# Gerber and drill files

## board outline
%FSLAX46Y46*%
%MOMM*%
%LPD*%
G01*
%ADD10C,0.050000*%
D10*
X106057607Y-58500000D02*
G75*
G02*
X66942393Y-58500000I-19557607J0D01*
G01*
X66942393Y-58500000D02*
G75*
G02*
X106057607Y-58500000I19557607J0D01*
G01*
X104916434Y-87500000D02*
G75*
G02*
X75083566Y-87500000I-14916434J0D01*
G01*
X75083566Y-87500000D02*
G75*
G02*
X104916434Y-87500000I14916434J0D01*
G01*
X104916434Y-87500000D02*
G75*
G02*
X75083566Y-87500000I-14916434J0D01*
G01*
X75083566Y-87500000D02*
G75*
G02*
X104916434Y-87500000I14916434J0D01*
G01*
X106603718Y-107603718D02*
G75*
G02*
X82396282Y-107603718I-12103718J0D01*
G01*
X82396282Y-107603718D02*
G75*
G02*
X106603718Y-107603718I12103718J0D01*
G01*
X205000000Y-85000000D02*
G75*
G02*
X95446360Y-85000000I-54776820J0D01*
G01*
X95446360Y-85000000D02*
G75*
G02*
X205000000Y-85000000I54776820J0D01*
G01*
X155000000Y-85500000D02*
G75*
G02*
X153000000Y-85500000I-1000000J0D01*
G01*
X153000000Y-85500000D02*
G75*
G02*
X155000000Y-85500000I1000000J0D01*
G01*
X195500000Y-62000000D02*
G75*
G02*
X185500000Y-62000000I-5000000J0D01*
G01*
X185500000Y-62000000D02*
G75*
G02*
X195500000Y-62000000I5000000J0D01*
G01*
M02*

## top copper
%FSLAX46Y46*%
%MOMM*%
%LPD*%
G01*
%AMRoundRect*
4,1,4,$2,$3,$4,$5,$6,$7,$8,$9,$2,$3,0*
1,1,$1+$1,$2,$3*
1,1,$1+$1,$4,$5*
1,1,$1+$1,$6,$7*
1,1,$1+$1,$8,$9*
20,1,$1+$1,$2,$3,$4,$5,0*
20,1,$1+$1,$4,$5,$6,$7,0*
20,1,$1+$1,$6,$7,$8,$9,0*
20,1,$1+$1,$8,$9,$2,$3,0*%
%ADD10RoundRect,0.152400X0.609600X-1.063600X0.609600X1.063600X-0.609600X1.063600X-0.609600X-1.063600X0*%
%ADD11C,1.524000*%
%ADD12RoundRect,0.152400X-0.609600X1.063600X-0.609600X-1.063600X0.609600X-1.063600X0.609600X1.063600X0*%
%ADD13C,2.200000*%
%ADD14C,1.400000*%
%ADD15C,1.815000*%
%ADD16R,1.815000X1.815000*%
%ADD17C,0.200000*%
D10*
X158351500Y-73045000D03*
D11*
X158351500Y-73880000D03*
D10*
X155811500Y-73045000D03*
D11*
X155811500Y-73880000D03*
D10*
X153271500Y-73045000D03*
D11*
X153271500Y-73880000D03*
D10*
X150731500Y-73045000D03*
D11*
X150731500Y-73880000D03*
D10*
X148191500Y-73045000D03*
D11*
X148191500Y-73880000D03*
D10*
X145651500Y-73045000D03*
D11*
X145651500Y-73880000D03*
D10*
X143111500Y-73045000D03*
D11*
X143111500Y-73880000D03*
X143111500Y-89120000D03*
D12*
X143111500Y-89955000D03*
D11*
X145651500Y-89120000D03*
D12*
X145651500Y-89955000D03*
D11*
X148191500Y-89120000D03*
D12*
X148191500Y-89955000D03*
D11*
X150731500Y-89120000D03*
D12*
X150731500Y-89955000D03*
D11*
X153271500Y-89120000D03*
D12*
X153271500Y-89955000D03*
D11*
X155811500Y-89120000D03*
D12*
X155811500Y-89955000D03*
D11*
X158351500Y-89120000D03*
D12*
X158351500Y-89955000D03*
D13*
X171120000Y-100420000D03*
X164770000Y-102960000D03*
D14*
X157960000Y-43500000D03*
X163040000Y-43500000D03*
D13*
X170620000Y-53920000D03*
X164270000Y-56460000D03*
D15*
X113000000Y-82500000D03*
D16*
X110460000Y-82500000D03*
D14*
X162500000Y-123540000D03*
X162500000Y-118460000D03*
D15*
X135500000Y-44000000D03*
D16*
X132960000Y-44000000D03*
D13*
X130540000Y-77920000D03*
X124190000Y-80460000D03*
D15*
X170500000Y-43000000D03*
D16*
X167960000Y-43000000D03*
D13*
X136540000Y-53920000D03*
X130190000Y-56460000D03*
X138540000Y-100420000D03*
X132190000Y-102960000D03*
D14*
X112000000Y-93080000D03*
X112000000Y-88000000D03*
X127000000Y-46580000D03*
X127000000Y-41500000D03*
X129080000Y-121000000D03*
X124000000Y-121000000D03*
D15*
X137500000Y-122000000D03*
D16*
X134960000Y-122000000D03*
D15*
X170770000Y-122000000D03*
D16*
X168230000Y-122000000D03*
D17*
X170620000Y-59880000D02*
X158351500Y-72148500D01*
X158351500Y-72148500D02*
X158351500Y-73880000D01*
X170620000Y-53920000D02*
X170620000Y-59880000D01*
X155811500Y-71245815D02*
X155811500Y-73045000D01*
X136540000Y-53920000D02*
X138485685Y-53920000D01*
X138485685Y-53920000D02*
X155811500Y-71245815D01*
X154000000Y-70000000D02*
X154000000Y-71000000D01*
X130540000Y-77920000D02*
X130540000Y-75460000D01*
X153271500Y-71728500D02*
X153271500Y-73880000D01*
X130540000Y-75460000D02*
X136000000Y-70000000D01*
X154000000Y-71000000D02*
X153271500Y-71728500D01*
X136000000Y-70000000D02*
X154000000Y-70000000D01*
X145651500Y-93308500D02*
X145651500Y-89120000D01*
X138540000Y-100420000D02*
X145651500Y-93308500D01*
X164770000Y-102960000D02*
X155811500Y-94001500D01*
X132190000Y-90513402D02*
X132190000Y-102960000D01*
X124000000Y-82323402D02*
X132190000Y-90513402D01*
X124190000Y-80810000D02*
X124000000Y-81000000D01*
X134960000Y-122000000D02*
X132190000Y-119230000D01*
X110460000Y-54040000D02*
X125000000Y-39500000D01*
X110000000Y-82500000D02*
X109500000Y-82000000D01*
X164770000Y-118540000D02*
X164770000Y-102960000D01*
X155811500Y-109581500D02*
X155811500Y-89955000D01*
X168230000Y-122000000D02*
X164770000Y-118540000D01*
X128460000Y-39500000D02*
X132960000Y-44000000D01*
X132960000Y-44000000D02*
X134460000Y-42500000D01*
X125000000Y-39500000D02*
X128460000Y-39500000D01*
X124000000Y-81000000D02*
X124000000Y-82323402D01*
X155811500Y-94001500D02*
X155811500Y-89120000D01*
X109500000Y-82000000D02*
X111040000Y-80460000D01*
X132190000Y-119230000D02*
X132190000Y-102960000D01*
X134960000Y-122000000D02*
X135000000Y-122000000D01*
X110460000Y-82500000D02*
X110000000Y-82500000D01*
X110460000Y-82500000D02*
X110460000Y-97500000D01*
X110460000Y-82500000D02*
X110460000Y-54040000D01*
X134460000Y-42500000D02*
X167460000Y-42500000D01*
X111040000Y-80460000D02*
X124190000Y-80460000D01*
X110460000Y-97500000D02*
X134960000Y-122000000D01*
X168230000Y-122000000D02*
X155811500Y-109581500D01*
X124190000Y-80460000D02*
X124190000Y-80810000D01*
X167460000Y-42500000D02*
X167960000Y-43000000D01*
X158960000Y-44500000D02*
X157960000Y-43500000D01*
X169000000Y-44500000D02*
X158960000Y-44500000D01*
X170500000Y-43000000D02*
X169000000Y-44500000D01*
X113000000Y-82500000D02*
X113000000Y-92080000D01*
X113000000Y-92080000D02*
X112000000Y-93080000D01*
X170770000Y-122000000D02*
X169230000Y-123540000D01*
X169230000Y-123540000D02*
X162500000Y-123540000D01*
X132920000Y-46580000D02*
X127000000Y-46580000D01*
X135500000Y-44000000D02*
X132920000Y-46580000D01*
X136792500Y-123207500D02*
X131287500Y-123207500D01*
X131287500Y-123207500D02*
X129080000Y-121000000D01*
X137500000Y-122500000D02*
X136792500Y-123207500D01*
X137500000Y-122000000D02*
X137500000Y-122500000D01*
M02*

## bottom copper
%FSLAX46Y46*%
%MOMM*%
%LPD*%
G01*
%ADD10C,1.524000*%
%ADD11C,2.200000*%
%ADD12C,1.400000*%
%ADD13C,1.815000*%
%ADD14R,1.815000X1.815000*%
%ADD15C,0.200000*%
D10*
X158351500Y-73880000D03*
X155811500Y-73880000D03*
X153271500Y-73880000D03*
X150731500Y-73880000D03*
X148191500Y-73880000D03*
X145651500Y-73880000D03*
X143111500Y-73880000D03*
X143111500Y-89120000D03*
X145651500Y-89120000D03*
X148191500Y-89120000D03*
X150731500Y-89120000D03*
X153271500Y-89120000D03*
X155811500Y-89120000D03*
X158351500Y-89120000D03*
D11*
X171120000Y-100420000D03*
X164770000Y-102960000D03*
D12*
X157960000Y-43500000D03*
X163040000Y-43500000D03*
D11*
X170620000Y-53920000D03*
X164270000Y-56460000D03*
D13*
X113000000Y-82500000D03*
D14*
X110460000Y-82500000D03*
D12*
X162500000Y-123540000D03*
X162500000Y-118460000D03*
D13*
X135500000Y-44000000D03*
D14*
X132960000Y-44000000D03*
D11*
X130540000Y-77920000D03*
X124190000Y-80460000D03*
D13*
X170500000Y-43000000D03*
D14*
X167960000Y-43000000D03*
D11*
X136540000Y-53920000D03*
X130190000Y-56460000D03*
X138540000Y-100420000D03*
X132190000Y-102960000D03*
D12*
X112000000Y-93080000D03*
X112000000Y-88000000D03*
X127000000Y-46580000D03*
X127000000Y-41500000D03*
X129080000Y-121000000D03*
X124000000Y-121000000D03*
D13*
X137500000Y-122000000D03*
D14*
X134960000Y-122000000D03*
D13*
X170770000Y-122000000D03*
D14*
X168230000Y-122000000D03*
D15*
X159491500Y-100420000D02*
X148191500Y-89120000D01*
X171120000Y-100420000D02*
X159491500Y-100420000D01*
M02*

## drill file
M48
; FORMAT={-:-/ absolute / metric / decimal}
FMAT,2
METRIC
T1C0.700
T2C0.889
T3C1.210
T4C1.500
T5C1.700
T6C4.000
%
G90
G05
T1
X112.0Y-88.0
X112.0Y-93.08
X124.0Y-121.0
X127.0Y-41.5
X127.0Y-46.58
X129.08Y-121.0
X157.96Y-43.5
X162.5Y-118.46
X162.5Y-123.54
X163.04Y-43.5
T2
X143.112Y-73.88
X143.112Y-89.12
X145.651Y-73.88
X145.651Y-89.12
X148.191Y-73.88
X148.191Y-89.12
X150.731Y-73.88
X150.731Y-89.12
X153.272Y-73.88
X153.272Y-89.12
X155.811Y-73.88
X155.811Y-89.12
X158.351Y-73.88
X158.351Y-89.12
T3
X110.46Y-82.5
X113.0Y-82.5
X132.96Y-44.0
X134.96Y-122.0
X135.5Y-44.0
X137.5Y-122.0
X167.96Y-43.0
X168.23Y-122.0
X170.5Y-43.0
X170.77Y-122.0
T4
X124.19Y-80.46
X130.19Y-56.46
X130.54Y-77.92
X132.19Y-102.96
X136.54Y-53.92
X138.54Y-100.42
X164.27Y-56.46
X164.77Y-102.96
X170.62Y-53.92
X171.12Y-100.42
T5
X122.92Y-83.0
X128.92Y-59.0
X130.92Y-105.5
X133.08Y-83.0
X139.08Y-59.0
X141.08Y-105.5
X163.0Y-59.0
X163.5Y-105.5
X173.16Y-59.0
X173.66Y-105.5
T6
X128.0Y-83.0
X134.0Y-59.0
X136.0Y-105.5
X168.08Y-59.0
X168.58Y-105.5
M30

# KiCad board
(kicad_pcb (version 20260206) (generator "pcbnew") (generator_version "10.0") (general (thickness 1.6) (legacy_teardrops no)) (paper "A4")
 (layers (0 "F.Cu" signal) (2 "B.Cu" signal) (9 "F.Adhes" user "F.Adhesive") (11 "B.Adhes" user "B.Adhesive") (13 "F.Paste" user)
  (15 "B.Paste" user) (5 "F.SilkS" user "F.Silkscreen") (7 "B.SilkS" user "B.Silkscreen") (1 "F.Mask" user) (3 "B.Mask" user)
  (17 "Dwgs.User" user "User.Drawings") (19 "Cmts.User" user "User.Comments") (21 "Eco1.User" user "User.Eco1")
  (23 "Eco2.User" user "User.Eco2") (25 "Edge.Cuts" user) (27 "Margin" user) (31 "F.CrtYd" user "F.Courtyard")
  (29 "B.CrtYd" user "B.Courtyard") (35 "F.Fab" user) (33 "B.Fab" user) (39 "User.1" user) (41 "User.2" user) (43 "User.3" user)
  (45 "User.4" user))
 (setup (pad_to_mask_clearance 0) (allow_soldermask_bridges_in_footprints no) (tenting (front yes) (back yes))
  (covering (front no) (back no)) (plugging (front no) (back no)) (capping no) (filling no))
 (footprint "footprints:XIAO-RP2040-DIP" (layer "F.Cu") (at 150.7315 81.5)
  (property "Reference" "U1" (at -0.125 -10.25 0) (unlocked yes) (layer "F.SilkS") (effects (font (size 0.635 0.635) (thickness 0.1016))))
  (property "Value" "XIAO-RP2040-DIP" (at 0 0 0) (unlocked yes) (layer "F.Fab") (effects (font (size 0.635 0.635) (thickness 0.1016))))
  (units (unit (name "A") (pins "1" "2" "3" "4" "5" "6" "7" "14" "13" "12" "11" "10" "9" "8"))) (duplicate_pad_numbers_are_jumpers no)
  (pad "1" smd roundrect (at 7.62 -8.455 90) (size 2.432 1.524) (layers "F.Cu" "F.Mask") (roundrect_rratio 0.1) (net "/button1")
   (thermal_bridge_angle 45))
  (pad "1" thru_hole circle (at 7.62 -7.62 90) (size 1.524 1.524) (drill 0.889) (layers "*.Cu" "*.Mask") (remove_unused_layers no)
   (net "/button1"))
  (pad "2" smd roundrect (at 5.08 -8.455 90) (size 2.432 1.524) (layers "F.Cu" "F.Mask") (roundrect_rratio 0.1) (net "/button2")
   (thermal_bridge_angle 45))
  (pad "2" thru_hole circle (at 5.08 -7.62 90) (size 1.524 1.524) (drill 0.889) (layers "*.Cu" "*.Mask") (remove_unused_layers no)
   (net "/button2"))
  (pad "3" smd roundrect (at 2.54 -8.455 90) (size 2.432 1.524) (layers "F.Cu" "F.Mask") (roundrect_rratio 0.1) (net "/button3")
   (thermal_bridge_angle 45))
  (pad "3" thru_hole circle (at 2.54 -7.62 90) (size 1.524 1.524) (drill 0.889) (layers "*.Cu" "*.Mask") (remove_unused_layers no)
   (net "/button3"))
  (pad "4" smd roundrect (at 0 -8.455 90) (size 2.432 1.524) (layers "F.Cu" "F.Mask") (roundrect_rratio 0.1) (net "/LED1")
   (thermal_bridge_angle 45))
  (pad "4" thru_hole circle (at 0 -7.62 90) (size 1.524 1.524) (drill 0.889) (layers "*.Cu" "*.Mask") (remove_unused_layers no)
   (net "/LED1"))
  (pad "5" smd roundrect (at -2.54 -8.455 90) (size 2.432 1.524) (layers "F.Cu" "F.Mask") (roundrect_rratio 0.1) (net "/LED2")
   (thermal_bridge_angle 45))
  (pad "5" thru_hole circle (at -2.54 -7.62 90) (size 1.524 1.524) (drill 0.889) (layers "*.Cu" "*.Mask") (remove_unused_layers no)
   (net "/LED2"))
  (pad "6" smd roundrect (at -5.08 -8.455 90) (size 2.432 1.524) (layers "F.Cu" "F.Mask") (roundrect_rratio 0.1) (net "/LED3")
   (thermal_bridge_angle 45))
  (pad "6" thru_hole circle (at -5.08 -7.62 90) (size 1.524 1.524) (drill 0.889) (layers "*.Cu" "*.Mask") (remove_unused_layers no)
   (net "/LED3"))
  (pad "7" smd roundrect (at -7.62 -8.455 90) (size 2.432 1.524) (layers "F.Cu" "F.Mask") (roundrect_rratio 0.1) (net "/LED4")
   (thermal_bridge_angle 45))
  (pad "7" thru_hole circle (at -7.62 -7.62 90) (size 1.524 1.524) (drill 0.889) (layers "*.Cu" "*.Mask") (remove_unused_layers no)
   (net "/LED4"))
  (pad "8" thru_hole circle (at -7.62 7.62 270) (size 1.524 1.524) (drill 0.889) (layers "*.Cu" "*.Mask") (remove_unused_layers no)
   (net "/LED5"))
  (pad "8" smd roundrect (at -7.62 8.455 270) (size 2.432 1.524) (layers "F.Cu" "F.Mask") (roundrect_rratio 0.1) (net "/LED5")
   (thermal_bridge_angle 45))
  (pad "9" thru_hole circle (at -5.08 7.62 270) (size 1.524 1.524) (drill 0.889) (layers "*.Cu" "*.Mask") (remove_unused_layers no)
   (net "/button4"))
  (pad "9" smd roundrect (at -5.08 8.455 270) (size 2.432 1.524) (layers "F.Cu" "F.Mask") (roundrect_rratio 0.1) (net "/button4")
   (thermal_bridge_angle 45))
  (pad "10" thru_hole circle (at -2.54 7.62 270) (size 1.524 1.524) (drill 0.889) (layers "*.Cu" "*.Mask") (remove_unused_layers no)
   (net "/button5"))
  (pad "10" smd roundrect (at -2.54 8.455 270) (size 2.432 1.524) (layers "F.Cu" "F.Mask") (roundrect_rratio 0.1) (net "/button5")
   (thermal_bridge_angle 45))
  (pad "11" thru_hole circle (at 0 7.62 270) (size 1.524 1.524) (drill 0.889) (layers "*.Cu" "*.Mask") (remove_unused_layers no)
   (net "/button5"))
  (pad "11" smd roundrect (at 0 8.455 270) (size 2.432 1.524) (layers "F.Cu" "F.Mask") (roundrect_rratio 0.1) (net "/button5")
   (thermal_bridge_angle 45))
  (pad "12" thru_hole circle (at 2.54 7.62 270) (size 1.524 1.524) (drill 0.889) (layers "*.Cu" "*.Mask") (remove_unused_layers no)
   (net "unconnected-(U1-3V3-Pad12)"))
  (pad "12" smd roundrect (at 2.54 8.455 270) (size 2.432 1.524) (layers "F.Cu" "F.Mask") (roundrect_rratio 0.1)
   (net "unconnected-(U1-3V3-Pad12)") (thermal_bridge_angle 45))
  (pad "13" thru_hole circle (at 5.08 7.62 270) (size 1.524 1.524) (drill 0.889) (layers "*.Cu" "*.Mask") (remove_unused_layers no)
   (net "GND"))
  (pad "13" smd roundrect (at 5.08 8.455 270) (size 2.432 1.524) (layers "F.Cu" "F.Mask") (roundrect_rratio 0.1) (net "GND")
   (thermal_bridge_angle 45))
  (pad "14" thru_hole circle (at 7.62 7.62 270) (size 1.524 1.524) (drill 0.889) (layers "*.Cu" "*.Mask") (remove_unused_layers no)
   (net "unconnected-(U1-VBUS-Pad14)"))
  (pad "14" smd roundrect (at 7.62 8.455 270) (size 2.432 1.524) (layers "F.Cu" "F.Mask") (roundrect_rratio 0.1)
   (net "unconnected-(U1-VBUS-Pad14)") (thermal_bridge_angle 45)))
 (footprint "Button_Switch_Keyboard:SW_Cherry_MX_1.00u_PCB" (layer "F.Cu") (at 171.12 100.42)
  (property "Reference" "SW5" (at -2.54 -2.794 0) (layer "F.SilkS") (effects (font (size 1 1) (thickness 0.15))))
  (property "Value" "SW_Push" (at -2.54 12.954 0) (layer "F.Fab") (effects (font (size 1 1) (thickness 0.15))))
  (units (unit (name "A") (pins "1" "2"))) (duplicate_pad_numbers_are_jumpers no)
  (pad "" np_thru_hole circle (at -7.62 5.08) (size 1.7 1.7) (drill 1.7) (layers "*.Cu" "*.Mask"))
  (pad "" np_thru_hole circle (at -2.54 5.08) (size 4 4) (drill 4) (layers "*.Cu" "*.Mask"))
  (pad "" np_thru_hole circle (at 2.54 5.08) (size 1.7 1.7) (drill 1.7) (layers "*.Cu" "*.Mask"))
  (pad "1" thru_hole circle (at 0 0) (size 2.2 2.2) (drill 1.5) (layers "*.Cu" "*.Mask") (remove_unused_layers no) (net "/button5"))
  (pad "2" thru_hole circle (at -6.35 2.54) (size 2.2 2.2) (drill 1.5) (layers "*.Cu" "*.Mask") (remove_unused_layers no) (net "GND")))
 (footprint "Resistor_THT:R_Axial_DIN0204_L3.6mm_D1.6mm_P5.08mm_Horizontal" (layer "F.Cu") (at 157.96 43.5)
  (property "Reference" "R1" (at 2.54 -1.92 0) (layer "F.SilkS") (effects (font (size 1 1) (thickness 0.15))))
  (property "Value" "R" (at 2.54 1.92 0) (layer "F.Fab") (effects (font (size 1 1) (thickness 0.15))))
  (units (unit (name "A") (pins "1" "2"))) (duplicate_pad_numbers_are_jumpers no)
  (pad "1" thru_hole circle (at 0 0) (size 1.4 1.4) (drill 0.7) (layers "*.Cu" "*.Mask") (remove_unused_layers no) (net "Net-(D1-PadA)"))
  (pad "2" thru_hole circle (at 5.08 0) (size 1.4 1.4) (drill 0.7) (layers "*.Cu" "*.Mask") (remove_unused_layers no) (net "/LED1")))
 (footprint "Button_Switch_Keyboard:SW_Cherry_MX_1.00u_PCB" (layer "F.Cu") (at 170.62 53.92)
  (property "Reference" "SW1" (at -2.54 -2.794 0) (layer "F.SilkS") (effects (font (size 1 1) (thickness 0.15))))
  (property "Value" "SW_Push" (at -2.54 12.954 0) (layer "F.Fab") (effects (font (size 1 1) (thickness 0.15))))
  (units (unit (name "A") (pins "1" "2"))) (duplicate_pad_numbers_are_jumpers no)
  (pad "" np_thru_hole circle (at -7.62 5.08) (size 1.7 1.7) (drill 1.7) (layers "*.Cu" "*.Mask"))
  (pad "" np_thru_hole circle (at -2.54 5.08) (size 4 4) (drill 4) (layers "*.Cu" "*.Mask"))
  (pad "" np_thru_hole circle (at 2.54 5.08) (size 1.7 1.7) (drill 1.7) (layers "*.Cu" "*.Mask"))
  (pad "1" thru_hole circle (at 0 0) (size 2.2 2.2) (drill 1.5) (layers "*.Cu" "*.Mask") (remove_unused_layers no) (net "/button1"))
  (pad "2" thru_hole circle (at -6.35 2.54) (size 2.2 2.2) (drill 1.5) (layers "*.Cu" "*.Mask") (remove_unused_layers no) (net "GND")))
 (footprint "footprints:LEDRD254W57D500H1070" (layer "F.Cu") (at 111.73 82.5)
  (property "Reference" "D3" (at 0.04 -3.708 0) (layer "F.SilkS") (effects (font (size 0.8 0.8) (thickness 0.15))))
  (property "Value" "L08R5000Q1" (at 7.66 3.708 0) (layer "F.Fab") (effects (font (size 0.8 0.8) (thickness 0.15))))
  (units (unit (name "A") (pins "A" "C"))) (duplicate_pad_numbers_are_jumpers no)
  (pad "A" thru_hole circle (at 1.27 0) (size 1.815 1.815) (drill 1.21) (layers "*.Cu" "*.Mask") (remove_unused_layers no)
   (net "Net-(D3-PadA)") (solder_mask_margin 0.102))
  (pad "C" thru_hole rect (at -1.27 0) (size 1.815 1.815) (drill 1.21) (layers "*.Cu" "*.Mask") (remove_unused_layers no) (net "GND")
   (solder_mask_margin 0.102)))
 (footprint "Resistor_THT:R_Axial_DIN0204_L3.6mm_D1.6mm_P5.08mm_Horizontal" (layer "F.Cu") (at 162.5 123.54 90)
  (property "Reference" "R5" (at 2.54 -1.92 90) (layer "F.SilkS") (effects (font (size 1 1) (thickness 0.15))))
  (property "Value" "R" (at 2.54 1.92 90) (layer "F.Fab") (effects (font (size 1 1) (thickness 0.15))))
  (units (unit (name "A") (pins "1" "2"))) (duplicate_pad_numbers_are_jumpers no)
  (pad "1" thru_hole circle (at 0 0 90) (size 1.4 1.4) (drill 0.7) (layers "*.Cu" "*.Mask") (remove_unused_layers no) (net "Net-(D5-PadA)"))
  (pad "2" thru_hole circle (at 5.08 0 90) (size 1.4 1.4) (drill 0.7) (layers "*.Cu" "*.Mask") (remove_unused_layers no) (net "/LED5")))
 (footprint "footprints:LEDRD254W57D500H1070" (layer "F.Cu") (at 134.23 44)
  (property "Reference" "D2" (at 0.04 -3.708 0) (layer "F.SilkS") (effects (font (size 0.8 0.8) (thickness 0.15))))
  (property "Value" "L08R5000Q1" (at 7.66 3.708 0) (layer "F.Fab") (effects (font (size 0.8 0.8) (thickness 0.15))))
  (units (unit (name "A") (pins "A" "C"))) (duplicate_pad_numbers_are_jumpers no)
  (pad "A" thru_hole circle (at 1.27 0) (size 1.815 1.815) (drill 1.21) (layers "*.Cu" "*.Mask") (remove_unused_layers no)
   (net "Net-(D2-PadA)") (solder_mask_margin 0.102))
  (pad "C" thru_hole rect (at -1.27 0) (size 1.815 1.815) (drill 1.21) (layers "*.Cu" "*.Mask") (remove_unused_layers no) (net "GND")
   (solder_mask_margin 0.102)))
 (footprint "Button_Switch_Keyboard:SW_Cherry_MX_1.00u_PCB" (layer "F.Cu") (at 130.54 77.92)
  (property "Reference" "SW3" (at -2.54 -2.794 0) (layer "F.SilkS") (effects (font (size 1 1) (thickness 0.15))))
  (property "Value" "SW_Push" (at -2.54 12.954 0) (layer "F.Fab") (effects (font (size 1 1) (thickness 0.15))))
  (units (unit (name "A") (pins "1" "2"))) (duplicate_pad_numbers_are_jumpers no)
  (pad "" np_thru_hole circle (at -7.62 5.08) (size 1.7 1.7) (drill 1.7) (layers "*.Cu" "*.Mask"))
  (pad "" np_thru_hole circle (at -2.54 5.08) (size 4 4) (drill 4) (layers "*.Cu" "*.Mask"))
  (pad "" np_thru_hole circle (at 2.54 5.08) (size 1.7 1.7) (drill 1.7) (layers "*.Cu" "*.Mask"))
  (pad "1" thru_hole circle (at 0 0) (size 2.2 2.2) (drill 1.5) (layers "*.Cu" "*.Mask") (remove_unused_layers no) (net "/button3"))
  (pad "2" thru_hole circle (at -6.35 2.54) (size 2.2 2.2) (drill 1.5) (layers "*.Cu" "*.Mask") (remove_unused_layers no) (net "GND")))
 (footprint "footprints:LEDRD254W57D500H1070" (layer "F.Cu") (at 169.23 43)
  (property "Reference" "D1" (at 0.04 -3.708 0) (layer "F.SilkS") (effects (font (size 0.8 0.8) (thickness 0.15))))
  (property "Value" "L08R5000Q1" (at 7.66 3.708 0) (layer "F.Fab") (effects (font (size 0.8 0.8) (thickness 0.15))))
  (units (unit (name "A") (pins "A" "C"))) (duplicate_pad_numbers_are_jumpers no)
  (pad "A" thru_hole circle (at 1.27 0) (size 1.815 1.815) (drill 1.21) (layers "*.Cu" "*.Mask") (remove_unused_layers no)
   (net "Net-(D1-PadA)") (solder_mask_margin 0.102))
  (pad "C" thru_hole rect (at -1.27 0) (size 1.815 1.815) (drill 1.21) (layers "*.Cu" "*.Mask") (remove_unused_layers no) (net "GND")
   (solder_mask_margin 0.102)))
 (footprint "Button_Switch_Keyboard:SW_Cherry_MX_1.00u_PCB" (layer "F.Cu") (at 136.54 53.92)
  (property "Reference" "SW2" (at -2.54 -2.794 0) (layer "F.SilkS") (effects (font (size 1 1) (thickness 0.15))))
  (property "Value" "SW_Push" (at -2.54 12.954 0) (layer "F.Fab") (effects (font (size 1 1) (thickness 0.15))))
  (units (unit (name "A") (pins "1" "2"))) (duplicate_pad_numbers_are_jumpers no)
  (pad "" np_thru_hole circle (at -7.62 5.08) (size 1.7 1.7) (drill 1.7) (layers "*.Cu" "*.Mask"))
  (pad "" np_thru_hole circle (at -2.54 5.08) (size 4 4) (drill 4) (layers "*.Cu" "*.Mask"))
  (pad "" np_thru_hole circle (at 2.54 5.08) (size 1.7 1.7) (drill 1.7) (layers "*.Cu" "*.Mask"))
  (pad "1" thru_hole circle (at 0 0) (size 2.2 2.2) (drill 1.5) (layers "*.Cu" "*.Mask") (remove_unused_layers no) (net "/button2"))
  (pad "2" thru_hole circle (at -6.35 2.54) (size 2.2 2.2) (drill 1.5) (layers "*.Cu" "*.Mask") (remove_unused_layers no) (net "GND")))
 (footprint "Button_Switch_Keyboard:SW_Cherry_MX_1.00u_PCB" (layer "F.Cu") (at 138.54 100.42)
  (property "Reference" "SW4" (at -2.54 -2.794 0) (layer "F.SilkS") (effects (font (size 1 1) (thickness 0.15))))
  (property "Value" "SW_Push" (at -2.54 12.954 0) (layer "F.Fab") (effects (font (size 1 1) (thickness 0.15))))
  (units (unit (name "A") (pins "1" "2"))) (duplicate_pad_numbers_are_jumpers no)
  (pad "" np_thru_hole circle (at -7.62 5.08) (size 1.7 1.7) (drill 1.7) (layers "*.Cu" "*.Mask"))
  (pad "" np_thru_hole circle (at -2.54 5.08) (size 4 4) (drill 4) (layers "*.Cu" "*.Mask"))
  (pad "" np_thru_hole circle (at 2.54 5.08) (size 1.7 1.7) (drill 1.7) (layers "*.Cu" "*.Mask"))
  (pad "1" thru_hole circle (at 0 0) (size 2.2 2.2) (drill 1.5) (layers "*.Cu" "*.Mask") (remove_unused_layers no) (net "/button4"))
  (pad "2" thru_hole circle (at -6.35 2.54) (size 2.2 2.2) (drill 1.5) (layers "*.Cu" "*.Mask") (remove_unused_layers no) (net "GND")))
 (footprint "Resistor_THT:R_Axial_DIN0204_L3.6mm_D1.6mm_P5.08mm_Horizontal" (layer "F.Cu") (at 112 93.08 90)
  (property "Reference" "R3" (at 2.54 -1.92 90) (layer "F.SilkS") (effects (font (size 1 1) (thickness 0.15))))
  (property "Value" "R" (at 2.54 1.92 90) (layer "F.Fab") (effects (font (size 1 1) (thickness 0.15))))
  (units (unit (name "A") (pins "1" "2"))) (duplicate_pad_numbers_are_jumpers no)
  (pad "1" thru_hole circle (at 0 0 90) (size 1.4 1.4) (drill 0.7) (layers "*.Cu" "*.Mask") (remove_unused_layers no) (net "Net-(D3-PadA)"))
  (pad "2" thru_hole circle (at 5.08 0 90) (size 1.4 1.4) (drill 0.7) (layers "*.Cu" "*.Mask") (remove_unused_layers no) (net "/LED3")))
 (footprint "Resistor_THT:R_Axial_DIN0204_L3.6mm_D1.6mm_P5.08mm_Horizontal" (layer "F.Cu") (at 127 46.58 90)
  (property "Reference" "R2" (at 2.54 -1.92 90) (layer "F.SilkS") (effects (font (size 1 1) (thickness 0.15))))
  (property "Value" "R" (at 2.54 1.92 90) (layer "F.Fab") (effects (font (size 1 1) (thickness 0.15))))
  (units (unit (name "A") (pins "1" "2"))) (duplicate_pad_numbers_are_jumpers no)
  (pad "1" thru_hole circle (at 0 0 90) (size 1.4 1.4) (drill 0.7) (layers "*.Cu" "*.Mask") (remove_unused_layers no) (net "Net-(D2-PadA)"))
  (pad "2" thru_hole circle (at 5.08 0 90) (size 1.4 1.4) (drill 0.7) (layers "*.Cu" "*.Mask") (remove_unused_layers no) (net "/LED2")))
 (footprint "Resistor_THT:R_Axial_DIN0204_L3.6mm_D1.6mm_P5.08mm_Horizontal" (layer "F.Cu") (at 129.08 121 180)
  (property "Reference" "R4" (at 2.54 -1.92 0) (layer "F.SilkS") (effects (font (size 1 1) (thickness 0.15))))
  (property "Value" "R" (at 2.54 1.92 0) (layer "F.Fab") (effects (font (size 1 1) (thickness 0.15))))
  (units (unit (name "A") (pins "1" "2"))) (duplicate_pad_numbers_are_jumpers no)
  (pad "1" thru_hole circle (at 0 0 180) (size 1.4 1.4) (drill 0.7) (layers "*.Cu" "*.Mask") (remove_unused_layers no) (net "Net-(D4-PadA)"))
  (pad "2" thru_hole circle (at 5.08 0 180) (size 1.4 1.4) (drill 0.7) (layers "*.Cu" "*.Mask") (remove_unused_layers no) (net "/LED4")))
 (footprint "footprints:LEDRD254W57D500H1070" (layer "F.Cu") (at 136.23 122)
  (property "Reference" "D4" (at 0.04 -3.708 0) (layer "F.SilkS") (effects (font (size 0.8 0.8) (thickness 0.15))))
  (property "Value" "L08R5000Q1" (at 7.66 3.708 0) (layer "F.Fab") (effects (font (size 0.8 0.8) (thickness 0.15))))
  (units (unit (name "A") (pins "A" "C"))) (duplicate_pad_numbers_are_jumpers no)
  (pad "A" thru_hole circle (at 1.27 0) (size 1.815 1.815) (drill 1.21) (layers "*.Cu" "*.Mask") (remove_unused_layers no)
   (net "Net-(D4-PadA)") (solder_mask_margin 0.102))
  (pad "C" thru_hole rect (at -1.27 0) (size 1.815 1.815) (drill 1.21) (layers "*.Cu" "*.Mask") (remove_unused_layers no) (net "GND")
   (solder_mask_margin 0.102)))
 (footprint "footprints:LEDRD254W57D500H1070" (layer "F.Cu") (at 169.5 122)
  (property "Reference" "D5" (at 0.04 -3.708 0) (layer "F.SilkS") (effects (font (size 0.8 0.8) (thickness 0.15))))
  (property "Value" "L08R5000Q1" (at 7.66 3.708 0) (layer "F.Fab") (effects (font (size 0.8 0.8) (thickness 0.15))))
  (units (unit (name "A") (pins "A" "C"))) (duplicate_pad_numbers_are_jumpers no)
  (pad "A" thru_hole circle (at 1.27 0) (size 1.815 1.815) (drill 1.21) (layers "*.Cu" "*.Mask") (remove_unused_layers no)
   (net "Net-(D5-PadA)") (solder_mask_margin 0.102))
  (pad "C" thru_hole rect (at -1.27 0) (size 1.815 1.815) (drill 1.21) (layers "*.Cu" "*.Mask") (remove_unused_layers no) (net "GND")
   (solder_mask_margin 0.102)))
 (gr_circle (center 86.5 58.5) (end 103 48) (stroke (width 0.05) (type default)) (fill no) (layer "Edge.Cuts"))
 (gr_circle (center 90 87.5) (end 90 72.583566) (stroke (width 0.05) (type default)) (fill no) (layer "Edge.Cuts"))
 (gr_circle (center 90 87.5) (end 93.5 73) (stroke (width 0.05) (type default)) (fill no) (layer "Edge.Cuts"))
 (gr_circle (center 94.5 107.603718) (end 102 98.103718) (stroke (width 0.05) (type default)) (fill no) (layer "Edge.Cuts"))
 (gr_circle (center 150.22318 85) (end 180.72318 39.5) (stroke (width 0.05) (type default)) (fill no) (layer "Edge.Cuts"))
 (gr_circle (center 154 85.5) (end 155 85.5) (stroke (width 0.05) (type default)) (fill no) (layer "Edge.Cuts"))
 (gr_circle (center 190.5 62) (end 194.5 59) (stroke (width 0.05) (type default)) (fill no) (layer "Edge.Cuts"))
 (segment (start 170.62 59.88) (end 158.3515 72.1485) (width 0.2) (layer "F.Cu") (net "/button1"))
 (segment (start 158.3515 72.1485) (end 158.3515 73.88) (width 0.2) (layer "F.Cu") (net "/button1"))
 (segment (start 170.62 53.92) (end 170.62 59.88) (width 0.2) (layer "F.Cu") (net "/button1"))
 (segment (start 155.8115 71.245815) (end 155.8115 73.045) (width 0.2) (layer "F.Cu") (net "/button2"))
 (segment (start 136.54 53.92) (end 138.485685 53.92) (width 0.2) (layer "F.Cu") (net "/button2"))
 (segment (start 138.485685 53.92) (end 155.8115 71.245815) (width 0.2) (layer "F.Cu") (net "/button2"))
 (segment (start 154 70) (end 154 71) (width 0.2) (layer "F.Cu") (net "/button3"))
 (segment (start 130.54 77.92) (end 130.54 75.46) (width 0.2) (layer "F.Cu") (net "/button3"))
 (segment (start 153.2715 71.7285) (end 153.2715 73.88) (width 0.2) (layer "F.Cu") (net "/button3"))
 (segment (start 130.54 75.46) (end 136 70) (width 0.2) (layer "F.Cu") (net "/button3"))
 (segment (start 154 71) (end 153.2715 71.7285) (width 0.2) (layer "F.Cu") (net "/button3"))
 (segment (start 136 70) (end 154 70) (width 0.2) (layer "F.Cu") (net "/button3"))
 (segment (start 145.6515 93.3085) (end 145.6515 89.12) (width 0.2) (layer "F.Cu") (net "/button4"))
 (segment (start 138.54 100.42) (end 145.6515 93.3085) (width 0.2) (layer "F.Cu") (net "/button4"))
 (segment (start 159.4915 100.42) (end 148.1915 89.12) (width 0.2) (layer "B.Cu") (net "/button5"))
 (segment (start 171.12 100.42) (end 159.4915 100.42) (width 0.2) (layer "B.Cu") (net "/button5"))
 (segment (start 164.77 102.96) (end 155.8115 94.0015) (width 0.2) (layer "F.Cu") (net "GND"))
 (segment (start 132.19 90.513402) (end 132.19 102.96) (width 0.2) (layer "F.Cu") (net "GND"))
 (segment (start 124 82.323402) (end 132.19 90.513402) (width 0.2) (layer "F.Cu") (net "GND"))
 (segment (start 124.19 80.81) (end 124 81) (width 0.2) (layer "F.Cu") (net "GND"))
 (segment (start 134.96 122) (end 132.19 119.23) (width 0.2) (layer "F.Cu") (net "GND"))
 (segment (start 110.46 54.04) (end 125 39.5) (width 0.2) (layer "F.Cu") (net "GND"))
 (segment (start 110 82.5) (end 109.5 82) (width 0.2) (layer "F.Cu") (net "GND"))
 (segment (start 164.77 118.54) (end 164.77 102.96) (width 0.2) (layer "F.Cu") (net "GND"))
 (segment (start 155.8115 109.5815) (end 155.8115 89.955) (width 0.2) (layer "F.Cu") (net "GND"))
 (segment (start 168.23 122) (end 164.77 118.54) (width 0.2) (layer "F.Cu") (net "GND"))
 (segment (start 128.46 39.5) (end 132.96 44) (width 0.2) (layer "F.Cu") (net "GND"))
 (segment (start 132.96 44) (end 134.46 42.5) (width 0.2) (layer "F.Cu") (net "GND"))
 (segment (start 125 39.5) (end 128.46 39.5) (width 0.2) (layer "F.Cu") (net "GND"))
 (segment (start 124 81) (end 124 82.323402) (width 0.2) (layer "F.Cu") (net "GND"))
 (segment (start 155.8115 94.0015) (end 155.8115 89.12) (width 0.2) (layer "F.Cu") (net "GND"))
 (segment (start 109.5 82) (end 111.04 80.46) (width 0.2) (layer "F.Cu") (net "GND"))
 (segment (start 132.19 119.23) (end 132.19 102.96) (width 0.2) (layer "F.Cu") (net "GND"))
 (segment (start 134.96 122) (end 135 122) (width 0.2) (layer "F.Cu") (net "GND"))
 (segment (start 110.46 82.5) (end 110 82.5) (width 0.2) (layer "F.Cu") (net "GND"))
 (segment (start 110.46 82.5) (end 110.46 97.5) (width 0.2) (layer "F.Cu") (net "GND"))
 (segment (start 110.46 82.5) (end 110.46 54.04) (width 0.2) (layer "F.Cu") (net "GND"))
 (segment (start 134.46 42.5) (end 167.46 42.5) (width 0.2) (layer "F.Cu") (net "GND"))
 (segment (start 111.04 80.46) (end 124.19 80.46) (width 0.2) (layer "F.Cu") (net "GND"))
 (segment (start 110.46 97.5) (end 134.96 122) (width 0.2) (layer "F.Cu") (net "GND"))
 (segment (start 168.23 122) (end 155.8115 109.5815) (width 0.2) (layer "F.Cu") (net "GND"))
 (segment (start 124.19 80.46) (end 124.19 80.81) (width 0.2) (layer "F.Cu") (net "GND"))
 (segment (start 167.46 42.5) (end 167.96 43) (width 0.2) (layer "F.Cu") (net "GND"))
 (segment (start 158.96 44.5) (end 157.96 43.5) (width 0.2) (layer "F.Cu") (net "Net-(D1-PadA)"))
 (segment (start 169 44.5) (end 158.96 44.5) (width 0.2) (layer "F.Cu") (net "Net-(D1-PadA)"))
 (segment (start 170.5 43) (end 169 44.5) (width 0.2) (layer "F.Cu") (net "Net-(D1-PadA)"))
 (segment (start 113 82.5) (end 113 92.08) (width 0.2) (layer "F.Cu") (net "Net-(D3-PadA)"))
 (segment (start 113 92.08) (end 112 93.08) (width 0.2) (layer "F.Cu") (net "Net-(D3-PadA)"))
 (segment (start 170.77 122) (end 169.23 123.54) (width 0.2) (layer "F.Cu") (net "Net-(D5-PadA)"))
 (segment (start 169.23 123.54) (end 162.5 123.54) (width 0.2) (layer "F.Cu") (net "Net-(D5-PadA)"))
 (segment (start 132.92 46.58) (end 127 46.58) (width 0.2) (layer "F.Cu") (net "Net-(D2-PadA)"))
 (segment (start 135.5 44) (end 132.92 46.58) (width 0.2) (layer "F.Cu") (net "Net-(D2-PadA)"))
 (segment (start 136.7925 123.2075) (end 131.2875 123.2075) (width 0.2) (layer "F.Cu") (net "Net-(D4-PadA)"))
 (segment (start 131.2875 123.2075) (end 129.08 121) (width 0.2) (layer "F.Cu") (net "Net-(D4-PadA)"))
 (segment (start 137.5 122.5) (end 136.7925 123.2075) (width 0.2) (layer "F.Cu") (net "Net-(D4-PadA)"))
 (segment (start 137.5 122) (end 137.5 122.5) (width 0.2) (layer "F.Cu") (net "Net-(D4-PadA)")))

